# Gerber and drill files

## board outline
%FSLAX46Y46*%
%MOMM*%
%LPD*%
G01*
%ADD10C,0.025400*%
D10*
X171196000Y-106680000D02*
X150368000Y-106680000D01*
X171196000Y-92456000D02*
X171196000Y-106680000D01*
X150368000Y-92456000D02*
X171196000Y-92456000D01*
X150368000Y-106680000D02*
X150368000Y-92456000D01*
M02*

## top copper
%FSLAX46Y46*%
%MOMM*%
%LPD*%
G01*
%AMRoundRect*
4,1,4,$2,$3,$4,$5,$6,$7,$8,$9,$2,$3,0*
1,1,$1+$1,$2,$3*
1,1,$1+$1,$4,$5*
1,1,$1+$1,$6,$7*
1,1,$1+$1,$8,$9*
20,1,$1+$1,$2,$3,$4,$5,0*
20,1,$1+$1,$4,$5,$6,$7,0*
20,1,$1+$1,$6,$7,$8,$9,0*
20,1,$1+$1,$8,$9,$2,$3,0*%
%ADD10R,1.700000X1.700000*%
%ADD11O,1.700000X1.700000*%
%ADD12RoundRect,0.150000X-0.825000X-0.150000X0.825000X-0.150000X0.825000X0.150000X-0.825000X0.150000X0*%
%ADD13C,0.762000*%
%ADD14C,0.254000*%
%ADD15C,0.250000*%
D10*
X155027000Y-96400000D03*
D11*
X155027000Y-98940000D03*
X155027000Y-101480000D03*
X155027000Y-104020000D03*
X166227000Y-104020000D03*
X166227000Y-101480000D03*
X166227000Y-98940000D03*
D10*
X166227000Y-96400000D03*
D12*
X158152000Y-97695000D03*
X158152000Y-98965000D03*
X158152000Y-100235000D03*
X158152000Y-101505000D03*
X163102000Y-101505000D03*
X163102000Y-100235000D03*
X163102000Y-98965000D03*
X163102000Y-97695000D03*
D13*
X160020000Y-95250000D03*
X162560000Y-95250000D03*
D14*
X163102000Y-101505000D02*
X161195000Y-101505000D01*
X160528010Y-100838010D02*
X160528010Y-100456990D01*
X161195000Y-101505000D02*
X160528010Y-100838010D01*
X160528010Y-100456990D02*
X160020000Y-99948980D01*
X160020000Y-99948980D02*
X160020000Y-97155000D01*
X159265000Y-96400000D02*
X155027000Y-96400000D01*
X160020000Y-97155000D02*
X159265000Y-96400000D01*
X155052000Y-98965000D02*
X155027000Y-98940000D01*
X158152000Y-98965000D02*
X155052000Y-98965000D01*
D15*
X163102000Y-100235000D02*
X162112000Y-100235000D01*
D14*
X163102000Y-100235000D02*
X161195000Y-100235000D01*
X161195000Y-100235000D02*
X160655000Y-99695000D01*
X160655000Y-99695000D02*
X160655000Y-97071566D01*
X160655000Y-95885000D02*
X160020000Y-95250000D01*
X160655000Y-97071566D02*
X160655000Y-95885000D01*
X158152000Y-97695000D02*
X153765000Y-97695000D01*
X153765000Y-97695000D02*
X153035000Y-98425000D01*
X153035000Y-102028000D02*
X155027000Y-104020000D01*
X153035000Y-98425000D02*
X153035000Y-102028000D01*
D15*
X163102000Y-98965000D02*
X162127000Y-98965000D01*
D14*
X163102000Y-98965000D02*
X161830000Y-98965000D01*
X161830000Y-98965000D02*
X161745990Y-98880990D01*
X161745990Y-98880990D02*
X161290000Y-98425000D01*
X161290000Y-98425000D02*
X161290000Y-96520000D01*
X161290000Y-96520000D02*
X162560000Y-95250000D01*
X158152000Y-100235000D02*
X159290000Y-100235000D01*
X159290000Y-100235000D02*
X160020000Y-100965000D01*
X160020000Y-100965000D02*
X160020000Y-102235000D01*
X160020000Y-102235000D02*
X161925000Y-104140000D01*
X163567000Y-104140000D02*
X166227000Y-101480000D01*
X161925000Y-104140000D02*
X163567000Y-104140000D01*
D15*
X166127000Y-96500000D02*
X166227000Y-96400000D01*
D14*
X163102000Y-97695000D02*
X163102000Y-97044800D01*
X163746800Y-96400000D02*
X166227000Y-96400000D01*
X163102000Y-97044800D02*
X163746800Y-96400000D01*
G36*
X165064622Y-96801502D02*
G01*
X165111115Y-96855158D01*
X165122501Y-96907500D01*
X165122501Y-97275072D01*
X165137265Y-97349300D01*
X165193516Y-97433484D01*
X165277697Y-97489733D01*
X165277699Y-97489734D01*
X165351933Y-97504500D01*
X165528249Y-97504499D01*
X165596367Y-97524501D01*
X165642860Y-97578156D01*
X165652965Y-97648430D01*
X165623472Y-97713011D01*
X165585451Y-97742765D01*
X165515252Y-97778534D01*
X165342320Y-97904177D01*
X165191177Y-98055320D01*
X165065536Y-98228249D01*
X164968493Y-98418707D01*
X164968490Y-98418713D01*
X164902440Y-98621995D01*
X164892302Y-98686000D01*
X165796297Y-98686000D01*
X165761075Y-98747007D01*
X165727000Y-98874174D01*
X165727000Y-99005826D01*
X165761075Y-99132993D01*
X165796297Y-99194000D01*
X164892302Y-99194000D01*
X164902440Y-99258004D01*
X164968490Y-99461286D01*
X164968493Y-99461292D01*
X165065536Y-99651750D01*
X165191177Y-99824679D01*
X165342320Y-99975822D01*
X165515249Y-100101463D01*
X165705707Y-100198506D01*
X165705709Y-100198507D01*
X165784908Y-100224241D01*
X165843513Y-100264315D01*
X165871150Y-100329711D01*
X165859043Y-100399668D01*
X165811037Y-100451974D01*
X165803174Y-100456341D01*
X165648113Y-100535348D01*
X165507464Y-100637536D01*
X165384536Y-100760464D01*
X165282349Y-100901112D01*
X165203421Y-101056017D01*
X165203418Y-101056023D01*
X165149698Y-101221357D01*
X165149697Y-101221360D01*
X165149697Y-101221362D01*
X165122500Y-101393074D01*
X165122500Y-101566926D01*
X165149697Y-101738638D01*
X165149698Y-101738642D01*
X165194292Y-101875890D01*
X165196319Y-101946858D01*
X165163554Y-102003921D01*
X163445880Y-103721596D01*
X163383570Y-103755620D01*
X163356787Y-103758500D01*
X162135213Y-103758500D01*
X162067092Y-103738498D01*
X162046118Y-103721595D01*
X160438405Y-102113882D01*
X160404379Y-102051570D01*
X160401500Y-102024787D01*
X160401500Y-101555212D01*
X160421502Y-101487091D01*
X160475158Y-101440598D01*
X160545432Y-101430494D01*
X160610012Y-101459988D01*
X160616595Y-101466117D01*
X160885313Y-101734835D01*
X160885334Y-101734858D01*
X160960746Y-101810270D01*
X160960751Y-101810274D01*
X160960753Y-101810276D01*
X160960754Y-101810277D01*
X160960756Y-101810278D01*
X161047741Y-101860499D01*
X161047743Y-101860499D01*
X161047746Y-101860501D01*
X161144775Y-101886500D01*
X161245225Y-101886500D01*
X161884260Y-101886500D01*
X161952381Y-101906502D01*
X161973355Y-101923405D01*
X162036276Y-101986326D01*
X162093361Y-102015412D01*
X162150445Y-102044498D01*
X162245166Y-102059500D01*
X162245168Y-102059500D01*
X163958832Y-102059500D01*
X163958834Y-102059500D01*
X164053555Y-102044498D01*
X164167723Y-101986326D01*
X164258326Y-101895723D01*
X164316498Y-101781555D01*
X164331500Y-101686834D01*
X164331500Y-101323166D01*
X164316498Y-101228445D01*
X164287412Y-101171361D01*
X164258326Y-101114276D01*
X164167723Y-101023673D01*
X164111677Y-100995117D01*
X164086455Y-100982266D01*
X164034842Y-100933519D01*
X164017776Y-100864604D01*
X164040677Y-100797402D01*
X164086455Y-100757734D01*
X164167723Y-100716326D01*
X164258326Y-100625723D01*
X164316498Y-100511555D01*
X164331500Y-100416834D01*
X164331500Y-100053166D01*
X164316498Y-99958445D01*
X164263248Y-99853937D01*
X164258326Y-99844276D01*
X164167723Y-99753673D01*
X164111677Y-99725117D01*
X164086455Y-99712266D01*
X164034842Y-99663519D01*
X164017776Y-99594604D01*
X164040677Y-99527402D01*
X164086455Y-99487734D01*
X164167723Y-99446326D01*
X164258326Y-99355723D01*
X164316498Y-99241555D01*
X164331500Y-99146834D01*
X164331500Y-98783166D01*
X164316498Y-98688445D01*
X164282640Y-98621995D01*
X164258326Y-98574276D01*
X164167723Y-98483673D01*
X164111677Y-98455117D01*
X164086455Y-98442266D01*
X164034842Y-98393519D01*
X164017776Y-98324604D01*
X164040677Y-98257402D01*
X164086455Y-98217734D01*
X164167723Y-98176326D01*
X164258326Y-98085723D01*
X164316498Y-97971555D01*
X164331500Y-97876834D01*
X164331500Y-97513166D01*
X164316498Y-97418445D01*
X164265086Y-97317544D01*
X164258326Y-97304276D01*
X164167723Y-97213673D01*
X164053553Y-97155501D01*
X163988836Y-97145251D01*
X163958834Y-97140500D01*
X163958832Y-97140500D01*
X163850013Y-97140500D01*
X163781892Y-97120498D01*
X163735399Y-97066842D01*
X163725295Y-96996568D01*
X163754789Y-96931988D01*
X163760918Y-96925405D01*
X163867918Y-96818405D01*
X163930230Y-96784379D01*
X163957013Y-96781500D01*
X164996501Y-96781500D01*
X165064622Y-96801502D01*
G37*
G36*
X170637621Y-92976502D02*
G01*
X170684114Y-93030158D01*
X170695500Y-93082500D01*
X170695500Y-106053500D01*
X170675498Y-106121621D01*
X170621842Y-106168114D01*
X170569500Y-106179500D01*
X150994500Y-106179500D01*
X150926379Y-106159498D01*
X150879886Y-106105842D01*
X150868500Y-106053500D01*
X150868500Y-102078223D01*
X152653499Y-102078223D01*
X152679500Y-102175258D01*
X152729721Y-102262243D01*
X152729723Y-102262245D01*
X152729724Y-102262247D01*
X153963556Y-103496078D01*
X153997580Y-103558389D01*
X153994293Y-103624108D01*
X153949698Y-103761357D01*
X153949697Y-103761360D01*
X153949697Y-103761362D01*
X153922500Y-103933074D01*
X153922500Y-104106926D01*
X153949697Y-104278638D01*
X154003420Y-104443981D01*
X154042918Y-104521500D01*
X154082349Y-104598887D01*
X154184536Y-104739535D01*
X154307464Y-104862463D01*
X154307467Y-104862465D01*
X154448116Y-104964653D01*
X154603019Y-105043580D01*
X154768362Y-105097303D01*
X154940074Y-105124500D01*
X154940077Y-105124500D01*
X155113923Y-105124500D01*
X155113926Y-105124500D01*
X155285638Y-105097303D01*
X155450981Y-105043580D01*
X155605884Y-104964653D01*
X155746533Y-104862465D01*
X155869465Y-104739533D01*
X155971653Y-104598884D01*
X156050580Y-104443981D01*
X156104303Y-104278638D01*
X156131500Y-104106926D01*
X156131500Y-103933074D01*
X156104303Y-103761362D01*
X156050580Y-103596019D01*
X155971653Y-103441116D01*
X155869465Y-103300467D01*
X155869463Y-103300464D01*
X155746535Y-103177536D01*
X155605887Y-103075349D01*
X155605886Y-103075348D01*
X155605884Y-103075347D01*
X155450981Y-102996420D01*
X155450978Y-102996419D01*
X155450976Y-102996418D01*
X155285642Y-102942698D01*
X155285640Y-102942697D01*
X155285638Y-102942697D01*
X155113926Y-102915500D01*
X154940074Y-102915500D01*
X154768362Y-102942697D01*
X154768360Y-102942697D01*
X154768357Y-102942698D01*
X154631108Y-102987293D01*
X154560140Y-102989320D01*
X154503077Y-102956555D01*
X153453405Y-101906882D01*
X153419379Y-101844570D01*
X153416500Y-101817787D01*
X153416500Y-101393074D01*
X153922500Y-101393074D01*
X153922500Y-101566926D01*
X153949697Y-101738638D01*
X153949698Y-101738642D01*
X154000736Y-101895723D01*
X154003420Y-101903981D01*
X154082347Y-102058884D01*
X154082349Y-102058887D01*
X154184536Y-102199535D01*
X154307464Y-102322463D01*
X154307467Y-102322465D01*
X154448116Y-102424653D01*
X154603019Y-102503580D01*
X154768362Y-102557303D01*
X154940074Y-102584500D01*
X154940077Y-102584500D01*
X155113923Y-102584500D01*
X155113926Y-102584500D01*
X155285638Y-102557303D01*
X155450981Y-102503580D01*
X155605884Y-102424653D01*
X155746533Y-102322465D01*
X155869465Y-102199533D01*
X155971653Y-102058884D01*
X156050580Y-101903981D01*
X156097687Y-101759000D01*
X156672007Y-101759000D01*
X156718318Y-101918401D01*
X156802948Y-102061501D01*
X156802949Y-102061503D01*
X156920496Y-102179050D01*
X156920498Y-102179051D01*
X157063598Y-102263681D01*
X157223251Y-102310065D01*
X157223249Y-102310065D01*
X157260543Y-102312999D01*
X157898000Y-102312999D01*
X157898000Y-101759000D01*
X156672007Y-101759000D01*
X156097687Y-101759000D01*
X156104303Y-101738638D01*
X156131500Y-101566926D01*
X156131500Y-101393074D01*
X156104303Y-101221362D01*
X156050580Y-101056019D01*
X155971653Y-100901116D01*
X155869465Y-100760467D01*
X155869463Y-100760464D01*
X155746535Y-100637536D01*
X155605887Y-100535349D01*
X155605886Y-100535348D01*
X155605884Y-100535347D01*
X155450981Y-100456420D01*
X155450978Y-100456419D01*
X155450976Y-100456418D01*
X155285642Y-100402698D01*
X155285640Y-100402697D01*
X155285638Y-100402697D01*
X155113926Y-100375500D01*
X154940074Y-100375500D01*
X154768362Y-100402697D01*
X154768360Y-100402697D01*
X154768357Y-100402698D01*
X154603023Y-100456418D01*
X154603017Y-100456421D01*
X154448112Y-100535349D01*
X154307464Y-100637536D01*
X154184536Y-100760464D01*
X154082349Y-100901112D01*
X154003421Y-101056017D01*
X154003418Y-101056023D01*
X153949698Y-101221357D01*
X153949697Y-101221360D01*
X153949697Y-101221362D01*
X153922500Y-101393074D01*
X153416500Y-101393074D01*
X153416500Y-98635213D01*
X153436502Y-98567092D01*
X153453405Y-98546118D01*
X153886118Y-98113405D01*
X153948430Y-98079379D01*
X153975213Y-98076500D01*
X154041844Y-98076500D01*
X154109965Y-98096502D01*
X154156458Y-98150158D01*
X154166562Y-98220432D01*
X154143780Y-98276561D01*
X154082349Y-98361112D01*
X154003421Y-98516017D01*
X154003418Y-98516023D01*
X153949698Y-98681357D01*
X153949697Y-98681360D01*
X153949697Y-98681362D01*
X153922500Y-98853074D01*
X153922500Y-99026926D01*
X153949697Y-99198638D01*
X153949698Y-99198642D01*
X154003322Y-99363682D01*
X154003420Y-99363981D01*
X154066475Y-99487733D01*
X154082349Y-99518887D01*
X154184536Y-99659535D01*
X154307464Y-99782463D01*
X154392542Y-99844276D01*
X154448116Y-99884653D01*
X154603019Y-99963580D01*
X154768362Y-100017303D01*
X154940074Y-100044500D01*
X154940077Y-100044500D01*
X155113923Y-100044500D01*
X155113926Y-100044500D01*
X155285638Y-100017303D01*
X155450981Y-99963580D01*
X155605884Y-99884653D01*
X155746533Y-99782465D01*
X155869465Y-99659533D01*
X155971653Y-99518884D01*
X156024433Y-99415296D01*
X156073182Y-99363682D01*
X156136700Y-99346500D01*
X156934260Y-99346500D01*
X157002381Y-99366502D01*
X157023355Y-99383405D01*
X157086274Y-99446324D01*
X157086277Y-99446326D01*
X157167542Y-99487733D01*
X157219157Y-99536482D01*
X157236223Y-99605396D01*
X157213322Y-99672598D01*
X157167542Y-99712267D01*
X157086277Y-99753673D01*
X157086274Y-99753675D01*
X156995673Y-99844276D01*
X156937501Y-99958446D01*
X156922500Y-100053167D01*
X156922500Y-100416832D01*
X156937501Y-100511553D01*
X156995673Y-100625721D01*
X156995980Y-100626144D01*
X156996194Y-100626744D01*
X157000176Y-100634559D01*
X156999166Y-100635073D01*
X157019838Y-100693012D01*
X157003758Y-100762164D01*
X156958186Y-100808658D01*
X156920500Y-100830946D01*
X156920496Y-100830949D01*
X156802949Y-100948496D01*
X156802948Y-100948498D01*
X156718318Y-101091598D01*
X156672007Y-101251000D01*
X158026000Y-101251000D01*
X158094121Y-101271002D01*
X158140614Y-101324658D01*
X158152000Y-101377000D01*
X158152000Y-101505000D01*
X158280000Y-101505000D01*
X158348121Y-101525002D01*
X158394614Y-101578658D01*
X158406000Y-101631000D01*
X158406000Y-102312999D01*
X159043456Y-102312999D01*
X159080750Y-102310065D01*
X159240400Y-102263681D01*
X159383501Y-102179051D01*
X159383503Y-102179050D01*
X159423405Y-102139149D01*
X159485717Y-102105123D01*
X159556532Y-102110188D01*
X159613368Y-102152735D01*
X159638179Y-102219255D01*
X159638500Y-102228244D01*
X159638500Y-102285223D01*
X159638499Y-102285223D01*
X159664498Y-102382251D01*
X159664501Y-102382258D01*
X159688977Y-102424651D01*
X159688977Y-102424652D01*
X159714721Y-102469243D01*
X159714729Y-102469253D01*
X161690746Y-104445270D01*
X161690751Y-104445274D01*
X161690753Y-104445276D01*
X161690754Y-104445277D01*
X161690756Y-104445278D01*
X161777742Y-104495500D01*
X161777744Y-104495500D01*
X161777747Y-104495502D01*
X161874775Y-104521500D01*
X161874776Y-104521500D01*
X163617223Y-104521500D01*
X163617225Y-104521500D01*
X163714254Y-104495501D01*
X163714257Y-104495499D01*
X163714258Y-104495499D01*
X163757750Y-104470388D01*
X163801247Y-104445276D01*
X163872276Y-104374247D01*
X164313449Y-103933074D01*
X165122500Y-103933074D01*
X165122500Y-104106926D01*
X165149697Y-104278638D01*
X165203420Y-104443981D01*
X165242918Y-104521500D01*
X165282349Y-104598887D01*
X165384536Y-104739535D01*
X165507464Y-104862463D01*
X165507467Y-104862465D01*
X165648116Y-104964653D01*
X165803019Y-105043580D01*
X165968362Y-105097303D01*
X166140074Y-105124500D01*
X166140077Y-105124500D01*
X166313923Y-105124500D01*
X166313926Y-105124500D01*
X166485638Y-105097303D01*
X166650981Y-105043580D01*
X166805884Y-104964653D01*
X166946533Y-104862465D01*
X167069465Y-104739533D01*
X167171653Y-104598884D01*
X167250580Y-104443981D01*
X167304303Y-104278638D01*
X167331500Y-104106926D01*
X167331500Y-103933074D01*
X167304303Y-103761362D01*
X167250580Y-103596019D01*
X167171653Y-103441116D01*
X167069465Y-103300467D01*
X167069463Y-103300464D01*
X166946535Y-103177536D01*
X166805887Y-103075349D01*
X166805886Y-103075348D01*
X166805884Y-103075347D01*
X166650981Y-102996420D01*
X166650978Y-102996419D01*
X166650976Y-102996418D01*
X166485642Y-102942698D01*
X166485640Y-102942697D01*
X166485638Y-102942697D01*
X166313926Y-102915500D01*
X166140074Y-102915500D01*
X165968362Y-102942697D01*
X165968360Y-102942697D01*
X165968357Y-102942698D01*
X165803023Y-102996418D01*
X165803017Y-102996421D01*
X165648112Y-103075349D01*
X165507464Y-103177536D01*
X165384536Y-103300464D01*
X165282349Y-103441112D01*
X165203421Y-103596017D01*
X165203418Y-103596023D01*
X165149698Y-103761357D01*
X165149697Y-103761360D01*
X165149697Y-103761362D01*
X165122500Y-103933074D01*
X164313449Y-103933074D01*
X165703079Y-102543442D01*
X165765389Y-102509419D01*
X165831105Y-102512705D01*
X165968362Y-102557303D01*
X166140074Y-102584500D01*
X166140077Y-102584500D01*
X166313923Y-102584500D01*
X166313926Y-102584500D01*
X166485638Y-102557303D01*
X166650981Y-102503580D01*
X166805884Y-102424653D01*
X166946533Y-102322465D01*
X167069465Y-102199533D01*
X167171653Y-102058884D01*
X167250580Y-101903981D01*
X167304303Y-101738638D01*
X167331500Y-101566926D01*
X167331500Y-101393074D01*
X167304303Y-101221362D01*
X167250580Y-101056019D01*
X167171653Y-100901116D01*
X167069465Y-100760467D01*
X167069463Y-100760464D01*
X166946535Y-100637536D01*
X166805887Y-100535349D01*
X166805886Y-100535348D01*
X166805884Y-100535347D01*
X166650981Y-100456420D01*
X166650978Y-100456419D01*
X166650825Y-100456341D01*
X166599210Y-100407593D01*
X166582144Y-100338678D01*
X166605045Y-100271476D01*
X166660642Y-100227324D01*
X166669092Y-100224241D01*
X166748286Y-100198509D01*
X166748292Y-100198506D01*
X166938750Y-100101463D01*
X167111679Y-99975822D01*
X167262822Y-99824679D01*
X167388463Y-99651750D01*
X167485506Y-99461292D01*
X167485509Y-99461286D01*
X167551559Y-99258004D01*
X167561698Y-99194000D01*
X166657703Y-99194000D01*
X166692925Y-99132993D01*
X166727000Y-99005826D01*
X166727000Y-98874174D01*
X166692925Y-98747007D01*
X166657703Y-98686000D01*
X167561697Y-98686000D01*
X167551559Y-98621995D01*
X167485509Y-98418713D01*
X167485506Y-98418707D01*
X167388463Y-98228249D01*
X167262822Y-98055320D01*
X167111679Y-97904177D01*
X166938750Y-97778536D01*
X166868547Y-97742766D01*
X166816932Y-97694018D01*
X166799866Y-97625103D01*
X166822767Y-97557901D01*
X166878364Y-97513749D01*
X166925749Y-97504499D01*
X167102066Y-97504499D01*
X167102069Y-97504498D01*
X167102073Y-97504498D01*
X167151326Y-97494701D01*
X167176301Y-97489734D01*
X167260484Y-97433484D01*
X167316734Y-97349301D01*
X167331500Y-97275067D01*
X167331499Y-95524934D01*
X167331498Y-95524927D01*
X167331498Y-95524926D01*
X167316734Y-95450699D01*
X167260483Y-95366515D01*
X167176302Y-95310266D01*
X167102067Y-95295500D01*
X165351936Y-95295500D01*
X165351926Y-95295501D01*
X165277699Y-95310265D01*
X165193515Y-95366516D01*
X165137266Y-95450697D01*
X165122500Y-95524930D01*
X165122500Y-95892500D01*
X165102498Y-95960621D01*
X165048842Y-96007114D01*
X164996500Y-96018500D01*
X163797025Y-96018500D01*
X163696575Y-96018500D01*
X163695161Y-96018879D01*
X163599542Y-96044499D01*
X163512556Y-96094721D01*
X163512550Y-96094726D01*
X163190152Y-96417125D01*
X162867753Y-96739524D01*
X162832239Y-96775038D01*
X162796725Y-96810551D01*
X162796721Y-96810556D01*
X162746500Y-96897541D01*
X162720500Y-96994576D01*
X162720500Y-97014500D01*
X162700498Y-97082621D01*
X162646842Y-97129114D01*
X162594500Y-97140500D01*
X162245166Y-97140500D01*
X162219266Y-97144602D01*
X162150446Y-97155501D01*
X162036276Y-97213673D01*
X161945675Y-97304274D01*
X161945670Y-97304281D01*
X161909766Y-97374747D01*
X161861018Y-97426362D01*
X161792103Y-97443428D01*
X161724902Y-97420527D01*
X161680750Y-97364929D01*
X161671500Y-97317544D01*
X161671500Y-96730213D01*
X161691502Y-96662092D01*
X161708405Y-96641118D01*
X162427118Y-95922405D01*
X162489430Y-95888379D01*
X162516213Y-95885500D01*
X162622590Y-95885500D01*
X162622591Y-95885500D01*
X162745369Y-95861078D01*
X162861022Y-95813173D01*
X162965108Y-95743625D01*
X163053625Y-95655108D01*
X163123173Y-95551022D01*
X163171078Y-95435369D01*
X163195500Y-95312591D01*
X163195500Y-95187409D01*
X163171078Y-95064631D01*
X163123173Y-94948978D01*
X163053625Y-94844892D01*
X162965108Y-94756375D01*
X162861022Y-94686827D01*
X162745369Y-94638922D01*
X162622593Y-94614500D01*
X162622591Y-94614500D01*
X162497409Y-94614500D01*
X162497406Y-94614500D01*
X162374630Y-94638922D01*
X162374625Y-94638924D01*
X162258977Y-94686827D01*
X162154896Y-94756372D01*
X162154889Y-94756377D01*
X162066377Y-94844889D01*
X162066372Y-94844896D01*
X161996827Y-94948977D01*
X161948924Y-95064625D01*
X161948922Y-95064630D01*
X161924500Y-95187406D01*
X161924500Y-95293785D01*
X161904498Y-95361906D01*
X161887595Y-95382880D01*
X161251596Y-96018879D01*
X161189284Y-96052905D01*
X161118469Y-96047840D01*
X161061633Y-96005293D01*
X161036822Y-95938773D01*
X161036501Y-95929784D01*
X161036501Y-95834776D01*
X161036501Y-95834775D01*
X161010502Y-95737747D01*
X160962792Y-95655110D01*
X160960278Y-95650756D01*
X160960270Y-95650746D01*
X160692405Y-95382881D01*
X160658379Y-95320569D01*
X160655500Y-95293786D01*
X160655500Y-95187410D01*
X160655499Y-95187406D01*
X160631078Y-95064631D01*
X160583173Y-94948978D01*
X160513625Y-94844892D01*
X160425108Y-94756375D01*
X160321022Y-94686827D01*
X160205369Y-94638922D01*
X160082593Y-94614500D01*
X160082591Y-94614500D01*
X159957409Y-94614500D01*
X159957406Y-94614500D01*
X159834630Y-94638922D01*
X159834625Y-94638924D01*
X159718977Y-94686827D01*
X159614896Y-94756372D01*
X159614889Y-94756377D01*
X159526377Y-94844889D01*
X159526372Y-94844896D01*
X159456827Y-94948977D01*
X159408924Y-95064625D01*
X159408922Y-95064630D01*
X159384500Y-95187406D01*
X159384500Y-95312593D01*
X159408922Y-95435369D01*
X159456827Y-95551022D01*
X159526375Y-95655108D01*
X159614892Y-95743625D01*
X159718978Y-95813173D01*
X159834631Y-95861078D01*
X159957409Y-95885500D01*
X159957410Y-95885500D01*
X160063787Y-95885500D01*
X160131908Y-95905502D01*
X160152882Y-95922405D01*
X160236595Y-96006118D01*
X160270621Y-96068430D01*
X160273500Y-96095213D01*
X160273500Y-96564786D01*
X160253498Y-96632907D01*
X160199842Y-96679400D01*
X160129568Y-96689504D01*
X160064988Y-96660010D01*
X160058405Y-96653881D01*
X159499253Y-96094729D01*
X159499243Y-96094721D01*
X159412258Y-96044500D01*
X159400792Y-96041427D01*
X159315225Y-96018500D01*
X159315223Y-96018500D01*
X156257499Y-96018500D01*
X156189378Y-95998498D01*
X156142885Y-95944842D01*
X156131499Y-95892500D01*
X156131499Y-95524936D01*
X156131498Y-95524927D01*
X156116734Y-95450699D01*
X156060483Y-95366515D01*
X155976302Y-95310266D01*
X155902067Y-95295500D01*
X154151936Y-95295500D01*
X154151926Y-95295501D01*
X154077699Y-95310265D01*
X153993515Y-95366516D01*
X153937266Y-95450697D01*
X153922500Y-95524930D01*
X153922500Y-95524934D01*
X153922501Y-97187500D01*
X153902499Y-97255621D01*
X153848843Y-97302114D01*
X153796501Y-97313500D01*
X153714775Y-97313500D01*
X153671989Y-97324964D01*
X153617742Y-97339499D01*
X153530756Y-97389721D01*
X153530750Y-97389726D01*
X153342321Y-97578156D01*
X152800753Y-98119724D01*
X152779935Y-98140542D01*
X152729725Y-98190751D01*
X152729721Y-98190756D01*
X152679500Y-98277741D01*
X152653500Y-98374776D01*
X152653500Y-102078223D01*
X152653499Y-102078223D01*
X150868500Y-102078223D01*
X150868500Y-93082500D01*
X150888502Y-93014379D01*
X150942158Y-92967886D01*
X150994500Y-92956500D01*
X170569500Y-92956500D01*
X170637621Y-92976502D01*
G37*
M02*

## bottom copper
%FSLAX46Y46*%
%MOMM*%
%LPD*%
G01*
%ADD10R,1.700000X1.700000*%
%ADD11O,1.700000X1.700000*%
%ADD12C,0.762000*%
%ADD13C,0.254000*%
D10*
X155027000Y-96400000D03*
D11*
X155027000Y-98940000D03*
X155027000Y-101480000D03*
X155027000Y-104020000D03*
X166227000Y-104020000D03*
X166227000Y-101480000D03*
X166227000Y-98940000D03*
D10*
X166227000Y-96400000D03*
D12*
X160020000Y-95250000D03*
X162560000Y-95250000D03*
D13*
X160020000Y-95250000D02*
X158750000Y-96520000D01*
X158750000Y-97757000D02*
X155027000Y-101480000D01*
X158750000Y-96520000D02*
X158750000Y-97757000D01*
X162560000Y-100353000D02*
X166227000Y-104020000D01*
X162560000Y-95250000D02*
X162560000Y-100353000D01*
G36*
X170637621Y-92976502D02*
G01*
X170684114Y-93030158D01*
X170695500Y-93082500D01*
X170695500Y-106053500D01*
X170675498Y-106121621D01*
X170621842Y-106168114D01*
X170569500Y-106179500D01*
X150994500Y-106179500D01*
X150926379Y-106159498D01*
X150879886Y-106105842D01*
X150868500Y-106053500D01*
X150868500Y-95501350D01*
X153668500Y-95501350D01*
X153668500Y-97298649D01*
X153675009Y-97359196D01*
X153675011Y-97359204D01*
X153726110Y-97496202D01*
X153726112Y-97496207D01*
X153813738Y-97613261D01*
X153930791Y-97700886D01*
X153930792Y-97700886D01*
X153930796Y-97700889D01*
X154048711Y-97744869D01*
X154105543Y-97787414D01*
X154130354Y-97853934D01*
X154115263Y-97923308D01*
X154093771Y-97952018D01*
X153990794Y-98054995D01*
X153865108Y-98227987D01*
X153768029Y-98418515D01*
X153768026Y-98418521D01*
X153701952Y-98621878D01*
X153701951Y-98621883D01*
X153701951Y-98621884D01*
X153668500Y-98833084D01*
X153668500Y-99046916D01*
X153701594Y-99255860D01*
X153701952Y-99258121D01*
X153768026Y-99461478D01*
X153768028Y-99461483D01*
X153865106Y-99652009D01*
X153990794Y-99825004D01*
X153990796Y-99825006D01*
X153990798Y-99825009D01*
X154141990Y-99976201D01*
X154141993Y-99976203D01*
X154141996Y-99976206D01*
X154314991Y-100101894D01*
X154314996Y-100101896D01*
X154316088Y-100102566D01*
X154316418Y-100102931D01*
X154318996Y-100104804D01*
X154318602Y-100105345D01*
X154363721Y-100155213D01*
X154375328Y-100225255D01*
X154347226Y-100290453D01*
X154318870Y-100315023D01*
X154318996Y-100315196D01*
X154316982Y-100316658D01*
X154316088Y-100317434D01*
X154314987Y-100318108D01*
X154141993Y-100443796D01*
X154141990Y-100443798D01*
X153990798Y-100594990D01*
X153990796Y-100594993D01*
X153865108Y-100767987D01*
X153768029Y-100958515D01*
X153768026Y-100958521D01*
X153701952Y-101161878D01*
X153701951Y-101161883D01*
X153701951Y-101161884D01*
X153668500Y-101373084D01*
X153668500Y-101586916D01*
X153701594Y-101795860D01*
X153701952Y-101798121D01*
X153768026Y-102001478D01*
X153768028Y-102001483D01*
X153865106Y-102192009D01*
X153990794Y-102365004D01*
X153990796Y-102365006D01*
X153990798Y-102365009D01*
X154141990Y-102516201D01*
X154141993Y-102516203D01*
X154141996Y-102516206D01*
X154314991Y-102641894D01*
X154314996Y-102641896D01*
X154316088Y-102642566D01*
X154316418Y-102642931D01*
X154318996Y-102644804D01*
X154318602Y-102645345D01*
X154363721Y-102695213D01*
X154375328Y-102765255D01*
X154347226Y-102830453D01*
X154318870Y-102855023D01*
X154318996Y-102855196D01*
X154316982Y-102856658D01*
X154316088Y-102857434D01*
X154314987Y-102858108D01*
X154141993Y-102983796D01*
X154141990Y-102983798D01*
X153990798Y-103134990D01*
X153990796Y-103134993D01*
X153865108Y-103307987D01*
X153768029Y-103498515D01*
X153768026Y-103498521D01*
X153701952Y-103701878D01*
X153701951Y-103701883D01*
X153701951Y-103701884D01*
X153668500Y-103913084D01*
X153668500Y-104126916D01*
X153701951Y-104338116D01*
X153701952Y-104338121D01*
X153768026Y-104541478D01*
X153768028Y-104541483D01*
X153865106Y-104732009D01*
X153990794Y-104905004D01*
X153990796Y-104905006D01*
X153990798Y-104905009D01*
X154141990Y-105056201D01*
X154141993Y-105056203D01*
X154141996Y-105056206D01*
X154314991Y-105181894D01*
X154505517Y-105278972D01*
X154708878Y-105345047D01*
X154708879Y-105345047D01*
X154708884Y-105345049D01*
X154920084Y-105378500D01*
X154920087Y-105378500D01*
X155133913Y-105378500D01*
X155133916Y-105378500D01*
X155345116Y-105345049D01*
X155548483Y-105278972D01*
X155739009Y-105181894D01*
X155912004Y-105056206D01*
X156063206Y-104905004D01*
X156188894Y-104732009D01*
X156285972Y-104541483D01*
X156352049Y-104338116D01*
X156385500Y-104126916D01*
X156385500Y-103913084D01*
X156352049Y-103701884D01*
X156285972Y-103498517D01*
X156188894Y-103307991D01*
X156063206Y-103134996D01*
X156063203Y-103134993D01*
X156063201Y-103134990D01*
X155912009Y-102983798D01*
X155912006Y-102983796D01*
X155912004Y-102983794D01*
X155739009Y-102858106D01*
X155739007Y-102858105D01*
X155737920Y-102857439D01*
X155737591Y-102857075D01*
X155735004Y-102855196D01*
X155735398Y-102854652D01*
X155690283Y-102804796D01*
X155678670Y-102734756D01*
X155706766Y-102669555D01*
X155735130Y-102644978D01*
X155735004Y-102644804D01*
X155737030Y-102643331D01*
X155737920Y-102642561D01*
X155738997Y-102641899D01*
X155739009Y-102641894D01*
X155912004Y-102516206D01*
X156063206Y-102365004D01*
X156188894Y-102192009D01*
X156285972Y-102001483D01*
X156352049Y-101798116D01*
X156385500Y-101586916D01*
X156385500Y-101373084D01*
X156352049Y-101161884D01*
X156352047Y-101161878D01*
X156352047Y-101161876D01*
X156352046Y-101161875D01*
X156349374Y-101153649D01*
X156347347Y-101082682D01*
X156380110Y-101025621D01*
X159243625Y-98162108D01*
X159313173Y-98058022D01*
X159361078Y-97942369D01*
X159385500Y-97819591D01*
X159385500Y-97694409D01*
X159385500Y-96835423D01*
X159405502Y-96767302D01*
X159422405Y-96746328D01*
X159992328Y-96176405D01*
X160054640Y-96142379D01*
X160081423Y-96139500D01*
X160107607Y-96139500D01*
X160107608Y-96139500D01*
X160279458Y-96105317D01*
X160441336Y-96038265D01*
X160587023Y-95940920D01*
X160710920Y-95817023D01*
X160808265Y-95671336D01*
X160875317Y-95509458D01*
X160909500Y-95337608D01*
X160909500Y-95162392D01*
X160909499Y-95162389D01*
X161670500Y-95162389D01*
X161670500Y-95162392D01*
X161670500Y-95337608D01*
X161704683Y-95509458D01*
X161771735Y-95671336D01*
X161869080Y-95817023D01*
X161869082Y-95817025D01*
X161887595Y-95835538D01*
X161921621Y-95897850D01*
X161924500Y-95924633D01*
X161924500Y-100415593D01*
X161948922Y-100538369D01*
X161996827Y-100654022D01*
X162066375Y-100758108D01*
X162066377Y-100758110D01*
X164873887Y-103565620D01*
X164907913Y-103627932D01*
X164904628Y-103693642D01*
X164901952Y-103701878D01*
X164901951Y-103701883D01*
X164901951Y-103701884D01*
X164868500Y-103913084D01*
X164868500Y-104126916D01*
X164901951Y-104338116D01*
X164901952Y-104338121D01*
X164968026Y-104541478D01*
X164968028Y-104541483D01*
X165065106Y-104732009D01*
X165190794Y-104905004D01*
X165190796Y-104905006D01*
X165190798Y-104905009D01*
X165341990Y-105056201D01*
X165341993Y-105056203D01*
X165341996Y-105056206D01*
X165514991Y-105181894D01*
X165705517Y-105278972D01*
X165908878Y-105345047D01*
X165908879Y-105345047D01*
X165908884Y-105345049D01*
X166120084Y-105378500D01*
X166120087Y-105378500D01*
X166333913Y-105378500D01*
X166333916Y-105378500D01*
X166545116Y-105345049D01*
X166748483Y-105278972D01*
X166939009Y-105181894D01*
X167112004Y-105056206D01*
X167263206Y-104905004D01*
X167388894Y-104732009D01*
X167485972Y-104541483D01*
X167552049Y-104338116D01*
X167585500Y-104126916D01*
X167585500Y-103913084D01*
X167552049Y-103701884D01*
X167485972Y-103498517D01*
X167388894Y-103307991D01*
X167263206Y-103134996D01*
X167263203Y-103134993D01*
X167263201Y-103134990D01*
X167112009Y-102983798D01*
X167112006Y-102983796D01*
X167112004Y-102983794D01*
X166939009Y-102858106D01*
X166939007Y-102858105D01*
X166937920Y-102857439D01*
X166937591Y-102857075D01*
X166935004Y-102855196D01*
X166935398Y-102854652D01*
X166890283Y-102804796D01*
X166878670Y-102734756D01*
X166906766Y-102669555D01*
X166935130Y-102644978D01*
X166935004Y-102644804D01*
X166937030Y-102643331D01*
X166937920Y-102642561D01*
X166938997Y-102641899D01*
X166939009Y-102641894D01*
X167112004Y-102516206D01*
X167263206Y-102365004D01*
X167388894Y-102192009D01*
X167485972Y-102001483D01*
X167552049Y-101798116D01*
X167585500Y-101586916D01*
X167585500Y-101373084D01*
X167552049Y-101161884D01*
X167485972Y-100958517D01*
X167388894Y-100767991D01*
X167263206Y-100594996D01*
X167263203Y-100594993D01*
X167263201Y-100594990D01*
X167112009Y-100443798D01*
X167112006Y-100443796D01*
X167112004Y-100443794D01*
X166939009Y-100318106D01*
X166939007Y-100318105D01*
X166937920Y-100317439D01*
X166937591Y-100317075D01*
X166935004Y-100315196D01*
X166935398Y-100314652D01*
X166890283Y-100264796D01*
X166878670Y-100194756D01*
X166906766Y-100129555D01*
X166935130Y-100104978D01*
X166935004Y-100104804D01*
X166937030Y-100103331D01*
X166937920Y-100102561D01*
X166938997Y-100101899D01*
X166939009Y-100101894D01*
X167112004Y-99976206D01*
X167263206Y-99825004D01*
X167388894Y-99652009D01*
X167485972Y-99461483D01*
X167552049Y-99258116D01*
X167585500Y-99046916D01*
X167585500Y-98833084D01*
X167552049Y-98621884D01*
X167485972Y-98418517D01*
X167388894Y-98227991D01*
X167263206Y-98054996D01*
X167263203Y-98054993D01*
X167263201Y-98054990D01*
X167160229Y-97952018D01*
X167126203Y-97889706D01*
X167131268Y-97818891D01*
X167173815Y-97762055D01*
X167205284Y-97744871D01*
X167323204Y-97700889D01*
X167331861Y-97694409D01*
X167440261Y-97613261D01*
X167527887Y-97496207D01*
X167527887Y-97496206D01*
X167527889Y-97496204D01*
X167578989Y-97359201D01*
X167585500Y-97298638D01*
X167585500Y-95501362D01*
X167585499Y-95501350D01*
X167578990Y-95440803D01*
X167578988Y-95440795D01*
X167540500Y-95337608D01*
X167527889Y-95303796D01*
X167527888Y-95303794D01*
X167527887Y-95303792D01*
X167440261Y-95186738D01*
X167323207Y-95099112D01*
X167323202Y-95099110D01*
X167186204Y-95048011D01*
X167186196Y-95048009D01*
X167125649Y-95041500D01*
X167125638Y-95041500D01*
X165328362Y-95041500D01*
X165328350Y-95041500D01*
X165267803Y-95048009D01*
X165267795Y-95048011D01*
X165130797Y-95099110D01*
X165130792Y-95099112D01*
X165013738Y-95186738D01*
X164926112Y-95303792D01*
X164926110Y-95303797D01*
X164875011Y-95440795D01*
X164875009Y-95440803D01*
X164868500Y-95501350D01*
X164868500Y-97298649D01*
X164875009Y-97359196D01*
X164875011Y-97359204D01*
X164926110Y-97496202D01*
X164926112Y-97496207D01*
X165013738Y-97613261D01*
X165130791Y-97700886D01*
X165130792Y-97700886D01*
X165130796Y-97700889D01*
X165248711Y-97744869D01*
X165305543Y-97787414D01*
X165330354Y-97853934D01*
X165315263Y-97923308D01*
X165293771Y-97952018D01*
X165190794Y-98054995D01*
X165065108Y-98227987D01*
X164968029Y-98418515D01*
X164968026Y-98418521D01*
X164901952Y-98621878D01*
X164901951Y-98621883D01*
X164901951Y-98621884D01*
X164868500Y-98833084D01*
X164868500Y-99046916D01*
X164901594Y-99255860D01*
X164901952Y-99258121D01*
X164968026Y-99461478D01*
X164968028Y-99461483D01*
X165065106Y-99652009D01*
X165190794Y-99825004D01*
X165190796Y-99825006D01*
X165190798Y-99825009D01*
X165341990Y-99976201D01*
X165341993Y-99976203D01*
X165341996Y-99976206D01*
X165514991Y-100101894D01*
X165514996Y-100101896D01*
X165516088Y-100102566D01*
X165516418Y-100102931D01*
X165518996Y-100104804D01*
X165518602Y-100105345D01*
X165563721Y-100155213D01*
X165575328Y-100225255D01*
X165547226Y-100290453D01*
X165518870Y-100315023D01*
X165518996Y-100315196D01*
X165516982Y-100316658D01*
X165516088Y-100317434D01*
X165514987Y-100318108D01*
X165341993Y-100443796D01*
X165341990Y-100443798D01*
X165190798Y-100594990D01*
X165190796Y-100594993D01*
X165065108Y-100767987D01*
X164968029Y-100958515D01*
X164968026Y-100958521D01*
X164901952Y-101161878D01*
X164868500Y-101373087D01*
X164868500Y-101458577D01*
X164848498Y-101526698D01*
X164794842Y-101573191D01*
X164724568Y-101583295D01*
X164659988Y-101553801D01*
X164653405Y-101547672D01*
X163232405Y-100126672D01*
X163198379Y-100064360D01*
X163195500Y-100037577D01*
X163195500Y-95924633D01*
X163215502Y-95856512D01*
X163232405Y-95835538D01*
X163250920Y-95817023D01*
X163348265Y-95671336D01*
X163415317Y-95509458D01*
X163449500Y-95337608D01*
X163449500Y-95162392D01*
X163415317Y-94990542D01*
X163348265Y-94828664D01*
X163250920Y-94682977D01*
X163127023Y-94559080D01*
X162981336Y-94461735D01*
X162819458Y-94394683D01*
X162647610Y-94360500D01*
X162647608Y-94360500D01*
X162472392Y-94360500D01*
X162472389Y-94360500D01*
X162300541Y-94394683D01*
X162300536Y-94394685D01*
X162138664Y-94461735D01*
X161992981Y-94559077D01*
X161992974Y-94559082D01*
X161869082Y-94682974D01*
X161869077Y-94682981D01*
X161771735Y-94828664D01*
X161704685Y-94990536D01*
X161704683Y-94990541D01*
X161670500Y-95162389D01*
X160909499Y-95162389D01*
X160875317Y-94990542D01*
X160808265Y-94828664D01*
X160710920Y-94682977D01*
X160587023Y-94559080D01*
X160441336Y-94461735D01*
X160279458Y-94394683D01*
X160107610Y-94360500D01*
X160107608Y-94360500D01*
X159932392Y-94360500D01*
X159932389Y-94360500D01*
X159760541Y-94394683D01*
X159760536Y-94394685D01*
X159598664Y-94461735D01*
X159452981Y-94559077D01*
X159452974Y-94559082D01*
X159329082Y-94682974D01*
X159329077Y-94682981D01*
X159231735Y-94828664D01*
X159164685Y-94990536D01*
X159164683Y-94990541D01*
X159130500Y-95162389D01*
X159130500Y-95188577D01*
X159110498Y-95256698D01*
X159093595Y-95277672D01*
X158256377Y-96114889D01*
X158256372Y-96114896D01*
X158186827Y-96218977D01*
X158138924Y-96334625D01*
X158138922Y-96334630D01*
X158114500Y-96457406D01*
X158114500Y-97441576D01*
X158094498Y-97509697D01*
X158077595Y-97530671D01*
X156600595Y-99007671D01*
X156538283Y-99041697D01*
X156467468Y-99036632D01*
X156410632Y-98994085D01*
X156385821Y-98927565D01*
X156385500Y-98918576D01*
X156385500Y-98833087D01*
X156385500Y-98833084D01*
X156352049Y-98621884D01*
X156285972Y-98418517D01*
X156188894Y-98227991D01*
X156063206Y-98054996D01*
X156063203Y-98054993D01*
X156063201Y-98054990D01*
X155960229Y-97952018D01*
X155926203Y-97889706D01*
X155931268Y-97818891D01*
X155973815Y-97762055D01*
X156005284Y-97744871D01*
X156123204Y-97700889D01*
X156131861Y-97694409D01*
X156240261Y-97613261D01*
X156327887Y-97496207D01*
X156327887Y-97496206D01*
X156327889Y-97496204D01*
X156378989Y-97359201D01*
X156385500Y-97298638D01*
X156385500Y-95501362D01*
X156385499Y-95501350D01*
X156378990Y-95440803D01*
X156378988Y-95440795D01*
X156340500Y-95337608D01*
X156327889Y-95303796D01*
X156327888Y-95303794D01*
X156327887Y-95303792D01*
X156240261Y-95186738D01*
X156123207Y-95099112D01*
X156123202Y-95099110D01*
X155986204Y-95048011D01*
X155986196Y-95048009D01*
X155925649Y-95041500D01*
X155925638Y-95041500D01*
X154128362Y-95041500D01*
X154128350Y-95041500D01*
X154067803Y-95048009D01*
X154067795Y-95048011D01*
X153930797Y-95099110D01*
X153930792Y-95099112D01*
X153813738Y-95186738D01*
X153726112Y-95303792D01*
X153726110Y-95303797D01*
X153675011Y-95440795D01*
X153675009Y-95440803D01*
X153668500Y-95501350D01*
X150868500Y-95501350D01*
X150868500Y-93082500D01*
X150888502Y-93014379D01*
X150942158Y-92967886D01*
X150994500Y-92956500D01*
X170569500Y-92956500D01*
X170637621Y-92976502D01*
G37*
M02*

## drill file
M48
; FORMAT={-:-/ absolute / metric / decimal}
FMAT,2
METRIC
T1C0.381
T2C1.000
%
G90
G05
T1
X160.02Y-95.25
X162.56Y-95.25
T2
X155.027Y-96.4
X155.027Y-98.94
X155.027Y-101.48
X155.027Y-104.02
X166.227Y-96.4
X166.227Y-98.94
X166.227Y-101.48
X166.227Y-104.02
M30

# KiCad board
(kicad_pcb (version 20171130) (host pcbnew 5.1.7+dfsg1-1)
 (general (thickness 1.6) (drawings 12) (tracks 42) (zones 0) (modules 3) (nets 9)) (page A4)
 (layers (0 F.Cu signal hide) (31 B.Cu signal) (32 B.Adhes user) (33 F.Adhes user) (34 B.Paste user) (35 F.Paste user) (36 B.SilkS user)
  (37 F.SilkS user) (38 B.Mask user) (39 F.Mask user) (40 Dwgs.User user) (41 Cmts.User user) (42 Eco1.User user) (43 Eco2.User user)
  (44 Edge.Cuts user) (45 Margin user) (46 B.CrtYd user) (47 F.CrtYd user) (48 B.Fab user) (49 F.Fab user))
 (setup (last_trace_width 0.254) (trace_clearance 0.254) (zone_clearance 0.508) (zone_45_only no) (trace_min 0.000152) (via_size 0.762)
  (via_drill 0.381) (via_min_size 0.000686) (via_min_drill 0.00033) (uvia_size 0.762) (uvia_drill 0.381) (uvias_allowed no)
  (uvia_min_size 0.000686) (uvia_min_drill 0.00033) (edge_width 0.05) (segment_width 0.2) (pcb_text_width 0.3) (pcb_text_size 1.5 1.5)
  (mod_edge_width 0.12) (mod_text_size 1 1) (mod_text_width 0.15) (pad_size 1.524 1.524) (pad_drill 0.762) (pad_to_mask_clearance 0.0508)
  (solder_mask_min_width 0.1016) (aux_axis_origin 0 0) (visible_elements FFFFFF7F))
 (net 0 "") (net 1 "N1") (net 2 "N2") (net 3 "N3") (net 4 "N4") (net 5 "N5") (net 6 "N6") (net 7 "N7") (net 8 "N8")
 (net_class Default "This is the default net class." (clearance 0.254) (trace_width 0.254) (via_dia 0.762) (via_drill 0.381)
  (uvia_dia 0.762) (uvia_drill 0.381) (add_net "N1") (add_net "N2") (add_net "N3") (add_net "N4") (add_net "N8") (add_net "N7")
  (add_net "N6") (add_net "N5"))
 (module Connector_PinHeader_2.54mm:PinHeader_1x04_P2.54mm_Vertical (layer F.Cu) (at 155.027 96.4)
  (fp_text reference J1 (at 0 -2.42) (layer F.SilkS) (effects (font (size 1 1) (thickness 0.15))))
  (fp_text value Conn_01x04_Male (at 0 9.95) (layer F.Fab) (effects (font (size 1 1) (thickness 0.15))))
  (pad 1 thru_hole rect (at 0 0) (size 1.7 1.7) (drill 1) (layers *.Cu *.Mask) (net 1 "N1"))
  (pad 2 thru_hole oval (at 0 2.54) (size 1.7 1.7) (drill 1) (layers *.Cu *.Mask) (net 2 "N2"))
  (pad 3 thru_hole oval (at 0 5.08) (size 1.7 1.7) (drill 1) (layers *.Cu *.Mask) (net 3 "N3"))
  (pad 4 thru_hole oval (at 0 7.62) (size 1.7 1.7) (drill 1) (layers *.Cu *.Mask) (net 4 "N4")))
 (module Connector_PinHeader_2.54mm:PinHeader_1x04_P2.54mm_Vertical (layer F.Cu) (at 166.227 96.4)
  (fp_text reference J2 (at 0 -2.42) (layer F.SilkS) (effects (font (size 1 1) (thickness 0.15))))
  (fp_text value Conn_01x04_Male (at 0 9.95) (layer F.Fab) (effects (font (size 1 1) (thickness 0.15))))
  (pad 4 thru_hole oval (at 0 7.62) (size 1.7 1.7) (drill 1) (layers *.Cu *.Mask) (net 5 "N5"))
  (pad 3 thru_hole oval (at 0 5.08) (size 1.7 1.7) (drill 1) (layers *.Cu *.Mask) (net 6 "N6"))
  (pad 2 thru_hole oval (at 0 2.54) (size 1.7 1.7) (drill 1) (layers *.Cu *.Mask) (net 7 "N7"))
  (pad 1 thru_hole rect (at 0 0) (size 1.7 1.7) (drill 1) (layers *.Cu *.Mask) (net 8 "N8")))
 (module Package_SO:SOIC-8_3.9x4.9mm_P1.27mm (layer F.Cu) (at 160.627 99.6)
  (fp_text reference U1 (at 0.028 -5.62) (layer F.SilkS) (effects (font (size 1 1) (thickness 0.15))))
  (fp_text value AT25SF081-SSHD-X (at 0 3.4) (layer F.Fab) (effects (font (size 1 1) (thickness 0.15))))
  (pad 1 smd roundrect (at -2.475 -1.905) (size 1.95 0.6) (layers F.Cu F.Paste F.Mask) (roundrect_rratio 0.25) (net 4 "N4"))
  (pad 2 smd roundrect (at -2.475 -0.635) (size 1.95 0.6) (layers F.Cu F.Paste F.Mask) (roundrect_rratio 0.25) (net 2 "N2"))
  (pad 3 smd roundrect (at -2.475 0.635) (size 1.95 0.6) (layers F.Cu F.Paste F.Mask) (roundrect_rratio 0.25) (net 6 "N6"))
  (pad 4 smd roundrect (at -2.475 1.905) (size 1.95 0.6) (layers F.Cu F.Paste F.Mask) (roundrect_rratio 0.25) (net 7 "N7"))
  (pad 5 smd roundrect (at 2.475 1.905) (size 1.95 0.6) (layers F.Cu F.Paste F.Mask) (roundrect_rratio 0.25) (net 1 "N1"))
  (pad 6 smd roundrect (at 2.475 0.635) (size 1.95 0.6) (layers F.Cu F.Paste F.Mask) (roundrect_rratio 0.25) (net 3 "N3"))
  (pad 7 smd roundrect (at 2.475 -0.635) (size 1.95 0.6) (layers F.Cu F.Paste F.Mask) (roundrect_rratio 0.25) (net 5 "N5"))
  (pad 8 smd roundrect (at 2.475 -1.905) (size 1.95 0.6) (layers F.Cu F.Paste F.Mask) (roundrect_rratio 0.25) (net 8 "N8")))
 (gr_line (start 171.196 106.68) (end 150.368 106.68) (layer Edge.Cuts) (width 0.0254))
 (gr_line (start 171.196 92.456) (end 171.196 106.68) (layer Edge.Cuts) (width 0.0254))
 (gr_line (start 150.368 92.456) (end 171.196 92.456) (layer Edge.Cuts) (width 0.0254))
 (gr_line (start 150.368 106.68) (end 150.368 92.456) (layer Edge.Cuts) (width 0.0254))
 (segment (start 163.102 101.505) (end 161.195 101.505) (width 0.254) (layer F.Cu) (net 1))
 (segment (start 160.52801 100.83801) (end 160.52801 100.45699) (width 0.254) (layer F.Cu) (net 1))
 (segment (start 161.195 101.505) (end 160.52801 100.83801) (width 0.254) (layer F.Cu) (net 1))
 (segment (start 160.52801 100.45699) (end 160.02 99.94898) (width 0.254) (layer F.Cu) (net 1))
 (segment (start 160.02 99.94898) (end 160.02 97.155) (width 0.254) (layer F.Cu) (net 1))
 (segment (start 159.265 96.4) (end 155.027 96.4) (width 0.254) (layer F.Cu) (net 1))
 (segment (start 160.02 97.155) (end 159.265 96.4) (width 0.254) (layer F.Cu) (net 1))
 (segment (start 155.052 98.965) (end 155.027 98.94) (width 0.254) (layer F.Cu) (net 2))
 (segment (start 158.152 98.965) (end 155.052 98.965) (width 0.254) (layer F.Cu) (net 2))
 (segment (start 163.102 100.235) (end 162.112 100.235) (width 0.25) (layer F.Cu) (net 3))
 (segment (start 163.102 100.235) (end 161.195 100.235) (width 0.254) (layer F.Cu) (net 3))
 (segment (start 161.195 100.235) (end 160.655 99.695) (width 0.254) (layer F.Cu) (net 3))
 (segment (start 160.655 99.695) (end 160.655 97.071566) (width 0.254) (layer F.Cu) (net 3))
 (via (at 160.02 95.25) (size 0.762) (drill 0.381) (layers F.Cu B.Cu) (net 3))
 (segment (start 160.655 95.885) (end 160.02 95.25) (width 0.254) (layer F.Cu) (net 3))
 (segment (start 160.655 97.071566) (end 160.655 95.885) (width 0.254) (layer F.Cu) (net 3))
 (segment (start 160.02 95.25) (end 158.75 96.52) (width 0.254) (layer B.Cu) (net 3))
 (segment (start 158.75 97.757) (end 155.027 101.48) (width 0.254) (layer B.Cu) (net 3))
 (segment (start 158.75 96.52) (end 158.75 97.757) (width 0.254) (layer B.Cu) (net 3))
 (segment (start 158.152 97.695) (end 153.765 97.695) (width 0.254) (layer F.Cu) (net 4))
 (segment (start 153.765 97.695) (end 153.035 98.425) (width 0.254) (layer F.Cu) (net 4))
 (segment (start 153.035 102.028) (end 155.027 104.02) (width 0.254) (layer F.Cu) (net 4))
 (segment (start 153.035 98.425) (end 153.035 102.028) (width 0.254) (layer F.Cu) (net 4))
 (segment (start 163.102 98.965) (end 162.127 98.965) (width 0.25) (layer F.Cu) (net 5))
 (segment (start 163.102 98.965) (end 161.83 98.965) (width 0.254) (layer F.Cu) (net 5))
 (segment (start 161.83 98.965) (end 161.74599 98.88099) (width 0.254) (layer F.Cu) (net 5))
 (segment (start 161.74599 98.88099) (end 161.29 98.425) (width 0.254) (layer F.Cu) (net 5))
 (segment (start 161.29 98.425) (end 161.29 96.52) (width 0.254) (layer F.Cu) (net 5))
 (via (at 162.56 95.25) (size 0.762) (drill 0.381) (layers F.Cu B.Cu) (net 5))
 (segment (start 161.29 96.52) (end 162.56 95.25) (width 0.254) (layer F.Cu) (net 5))
 (segment (start 162.56 100.353) (end 166.227 104.02) (width 0.254) (layer B.Cu) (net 5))
 (segment (start 162.56 95.25) (end 162.56 100.353) (width 0.254) (layer B.Cu) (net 5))
 (segment (start 158.152 100.235) (end 159.29 100.235) (width 0.254) (layer F.Cu) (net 6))
 (segment (start 159.29 100.235) (end 160.02 100.965) (width 0.254) (layer F.Cu) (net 6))
 (segment (start 160.02 100.965) (end 160.02 102.235) (width 0.254) (layer F.Cu) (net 6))
 (segment (start 160.02 102.235) (end 161.925 104.14) (width 0.254) (layer F.Cu) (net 6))
 (segment (start 163.567 104.14) (end 166.227 101.48) (width 0.254) (layer F.Cu) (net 6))
 (segment (start 161.925 104.14) (end 163.567 104.14) (width 0.254) (layer F.Cu) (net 6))
 (segment (start 166.127 96.5) (end 166.227 96.4) (width 0.25) (layer F.Cu) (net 8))
 (segment (start 163.102 97.695) (end 163.102 97.0448) (width 0.254) (layer F.Cu) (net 8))
 (segment (start 163.7468 96.4) (end 166.227 96.4) (width 0.254) (layer F.Cu) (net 8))
 (segment (start 163.102 97.0448) (end 163.7468 96.4) (width 0.254) (layer F.Cu) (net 8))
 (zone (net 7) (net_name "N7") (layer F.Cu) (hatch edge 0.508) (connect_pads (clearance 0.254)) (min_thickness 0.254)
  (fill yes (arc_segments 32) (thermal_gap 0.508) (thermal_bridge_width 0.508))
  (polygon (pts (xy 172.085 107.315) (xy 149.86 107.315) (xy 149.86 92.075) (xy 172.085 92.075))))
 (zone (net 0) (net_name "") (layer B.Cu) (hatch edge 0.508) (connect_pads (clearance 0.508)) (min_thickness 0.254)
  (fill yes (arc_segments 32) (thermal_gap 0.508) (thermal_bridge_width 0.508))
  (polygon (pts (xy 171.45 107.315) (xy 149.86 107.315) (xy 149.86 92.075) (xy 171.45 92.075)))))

